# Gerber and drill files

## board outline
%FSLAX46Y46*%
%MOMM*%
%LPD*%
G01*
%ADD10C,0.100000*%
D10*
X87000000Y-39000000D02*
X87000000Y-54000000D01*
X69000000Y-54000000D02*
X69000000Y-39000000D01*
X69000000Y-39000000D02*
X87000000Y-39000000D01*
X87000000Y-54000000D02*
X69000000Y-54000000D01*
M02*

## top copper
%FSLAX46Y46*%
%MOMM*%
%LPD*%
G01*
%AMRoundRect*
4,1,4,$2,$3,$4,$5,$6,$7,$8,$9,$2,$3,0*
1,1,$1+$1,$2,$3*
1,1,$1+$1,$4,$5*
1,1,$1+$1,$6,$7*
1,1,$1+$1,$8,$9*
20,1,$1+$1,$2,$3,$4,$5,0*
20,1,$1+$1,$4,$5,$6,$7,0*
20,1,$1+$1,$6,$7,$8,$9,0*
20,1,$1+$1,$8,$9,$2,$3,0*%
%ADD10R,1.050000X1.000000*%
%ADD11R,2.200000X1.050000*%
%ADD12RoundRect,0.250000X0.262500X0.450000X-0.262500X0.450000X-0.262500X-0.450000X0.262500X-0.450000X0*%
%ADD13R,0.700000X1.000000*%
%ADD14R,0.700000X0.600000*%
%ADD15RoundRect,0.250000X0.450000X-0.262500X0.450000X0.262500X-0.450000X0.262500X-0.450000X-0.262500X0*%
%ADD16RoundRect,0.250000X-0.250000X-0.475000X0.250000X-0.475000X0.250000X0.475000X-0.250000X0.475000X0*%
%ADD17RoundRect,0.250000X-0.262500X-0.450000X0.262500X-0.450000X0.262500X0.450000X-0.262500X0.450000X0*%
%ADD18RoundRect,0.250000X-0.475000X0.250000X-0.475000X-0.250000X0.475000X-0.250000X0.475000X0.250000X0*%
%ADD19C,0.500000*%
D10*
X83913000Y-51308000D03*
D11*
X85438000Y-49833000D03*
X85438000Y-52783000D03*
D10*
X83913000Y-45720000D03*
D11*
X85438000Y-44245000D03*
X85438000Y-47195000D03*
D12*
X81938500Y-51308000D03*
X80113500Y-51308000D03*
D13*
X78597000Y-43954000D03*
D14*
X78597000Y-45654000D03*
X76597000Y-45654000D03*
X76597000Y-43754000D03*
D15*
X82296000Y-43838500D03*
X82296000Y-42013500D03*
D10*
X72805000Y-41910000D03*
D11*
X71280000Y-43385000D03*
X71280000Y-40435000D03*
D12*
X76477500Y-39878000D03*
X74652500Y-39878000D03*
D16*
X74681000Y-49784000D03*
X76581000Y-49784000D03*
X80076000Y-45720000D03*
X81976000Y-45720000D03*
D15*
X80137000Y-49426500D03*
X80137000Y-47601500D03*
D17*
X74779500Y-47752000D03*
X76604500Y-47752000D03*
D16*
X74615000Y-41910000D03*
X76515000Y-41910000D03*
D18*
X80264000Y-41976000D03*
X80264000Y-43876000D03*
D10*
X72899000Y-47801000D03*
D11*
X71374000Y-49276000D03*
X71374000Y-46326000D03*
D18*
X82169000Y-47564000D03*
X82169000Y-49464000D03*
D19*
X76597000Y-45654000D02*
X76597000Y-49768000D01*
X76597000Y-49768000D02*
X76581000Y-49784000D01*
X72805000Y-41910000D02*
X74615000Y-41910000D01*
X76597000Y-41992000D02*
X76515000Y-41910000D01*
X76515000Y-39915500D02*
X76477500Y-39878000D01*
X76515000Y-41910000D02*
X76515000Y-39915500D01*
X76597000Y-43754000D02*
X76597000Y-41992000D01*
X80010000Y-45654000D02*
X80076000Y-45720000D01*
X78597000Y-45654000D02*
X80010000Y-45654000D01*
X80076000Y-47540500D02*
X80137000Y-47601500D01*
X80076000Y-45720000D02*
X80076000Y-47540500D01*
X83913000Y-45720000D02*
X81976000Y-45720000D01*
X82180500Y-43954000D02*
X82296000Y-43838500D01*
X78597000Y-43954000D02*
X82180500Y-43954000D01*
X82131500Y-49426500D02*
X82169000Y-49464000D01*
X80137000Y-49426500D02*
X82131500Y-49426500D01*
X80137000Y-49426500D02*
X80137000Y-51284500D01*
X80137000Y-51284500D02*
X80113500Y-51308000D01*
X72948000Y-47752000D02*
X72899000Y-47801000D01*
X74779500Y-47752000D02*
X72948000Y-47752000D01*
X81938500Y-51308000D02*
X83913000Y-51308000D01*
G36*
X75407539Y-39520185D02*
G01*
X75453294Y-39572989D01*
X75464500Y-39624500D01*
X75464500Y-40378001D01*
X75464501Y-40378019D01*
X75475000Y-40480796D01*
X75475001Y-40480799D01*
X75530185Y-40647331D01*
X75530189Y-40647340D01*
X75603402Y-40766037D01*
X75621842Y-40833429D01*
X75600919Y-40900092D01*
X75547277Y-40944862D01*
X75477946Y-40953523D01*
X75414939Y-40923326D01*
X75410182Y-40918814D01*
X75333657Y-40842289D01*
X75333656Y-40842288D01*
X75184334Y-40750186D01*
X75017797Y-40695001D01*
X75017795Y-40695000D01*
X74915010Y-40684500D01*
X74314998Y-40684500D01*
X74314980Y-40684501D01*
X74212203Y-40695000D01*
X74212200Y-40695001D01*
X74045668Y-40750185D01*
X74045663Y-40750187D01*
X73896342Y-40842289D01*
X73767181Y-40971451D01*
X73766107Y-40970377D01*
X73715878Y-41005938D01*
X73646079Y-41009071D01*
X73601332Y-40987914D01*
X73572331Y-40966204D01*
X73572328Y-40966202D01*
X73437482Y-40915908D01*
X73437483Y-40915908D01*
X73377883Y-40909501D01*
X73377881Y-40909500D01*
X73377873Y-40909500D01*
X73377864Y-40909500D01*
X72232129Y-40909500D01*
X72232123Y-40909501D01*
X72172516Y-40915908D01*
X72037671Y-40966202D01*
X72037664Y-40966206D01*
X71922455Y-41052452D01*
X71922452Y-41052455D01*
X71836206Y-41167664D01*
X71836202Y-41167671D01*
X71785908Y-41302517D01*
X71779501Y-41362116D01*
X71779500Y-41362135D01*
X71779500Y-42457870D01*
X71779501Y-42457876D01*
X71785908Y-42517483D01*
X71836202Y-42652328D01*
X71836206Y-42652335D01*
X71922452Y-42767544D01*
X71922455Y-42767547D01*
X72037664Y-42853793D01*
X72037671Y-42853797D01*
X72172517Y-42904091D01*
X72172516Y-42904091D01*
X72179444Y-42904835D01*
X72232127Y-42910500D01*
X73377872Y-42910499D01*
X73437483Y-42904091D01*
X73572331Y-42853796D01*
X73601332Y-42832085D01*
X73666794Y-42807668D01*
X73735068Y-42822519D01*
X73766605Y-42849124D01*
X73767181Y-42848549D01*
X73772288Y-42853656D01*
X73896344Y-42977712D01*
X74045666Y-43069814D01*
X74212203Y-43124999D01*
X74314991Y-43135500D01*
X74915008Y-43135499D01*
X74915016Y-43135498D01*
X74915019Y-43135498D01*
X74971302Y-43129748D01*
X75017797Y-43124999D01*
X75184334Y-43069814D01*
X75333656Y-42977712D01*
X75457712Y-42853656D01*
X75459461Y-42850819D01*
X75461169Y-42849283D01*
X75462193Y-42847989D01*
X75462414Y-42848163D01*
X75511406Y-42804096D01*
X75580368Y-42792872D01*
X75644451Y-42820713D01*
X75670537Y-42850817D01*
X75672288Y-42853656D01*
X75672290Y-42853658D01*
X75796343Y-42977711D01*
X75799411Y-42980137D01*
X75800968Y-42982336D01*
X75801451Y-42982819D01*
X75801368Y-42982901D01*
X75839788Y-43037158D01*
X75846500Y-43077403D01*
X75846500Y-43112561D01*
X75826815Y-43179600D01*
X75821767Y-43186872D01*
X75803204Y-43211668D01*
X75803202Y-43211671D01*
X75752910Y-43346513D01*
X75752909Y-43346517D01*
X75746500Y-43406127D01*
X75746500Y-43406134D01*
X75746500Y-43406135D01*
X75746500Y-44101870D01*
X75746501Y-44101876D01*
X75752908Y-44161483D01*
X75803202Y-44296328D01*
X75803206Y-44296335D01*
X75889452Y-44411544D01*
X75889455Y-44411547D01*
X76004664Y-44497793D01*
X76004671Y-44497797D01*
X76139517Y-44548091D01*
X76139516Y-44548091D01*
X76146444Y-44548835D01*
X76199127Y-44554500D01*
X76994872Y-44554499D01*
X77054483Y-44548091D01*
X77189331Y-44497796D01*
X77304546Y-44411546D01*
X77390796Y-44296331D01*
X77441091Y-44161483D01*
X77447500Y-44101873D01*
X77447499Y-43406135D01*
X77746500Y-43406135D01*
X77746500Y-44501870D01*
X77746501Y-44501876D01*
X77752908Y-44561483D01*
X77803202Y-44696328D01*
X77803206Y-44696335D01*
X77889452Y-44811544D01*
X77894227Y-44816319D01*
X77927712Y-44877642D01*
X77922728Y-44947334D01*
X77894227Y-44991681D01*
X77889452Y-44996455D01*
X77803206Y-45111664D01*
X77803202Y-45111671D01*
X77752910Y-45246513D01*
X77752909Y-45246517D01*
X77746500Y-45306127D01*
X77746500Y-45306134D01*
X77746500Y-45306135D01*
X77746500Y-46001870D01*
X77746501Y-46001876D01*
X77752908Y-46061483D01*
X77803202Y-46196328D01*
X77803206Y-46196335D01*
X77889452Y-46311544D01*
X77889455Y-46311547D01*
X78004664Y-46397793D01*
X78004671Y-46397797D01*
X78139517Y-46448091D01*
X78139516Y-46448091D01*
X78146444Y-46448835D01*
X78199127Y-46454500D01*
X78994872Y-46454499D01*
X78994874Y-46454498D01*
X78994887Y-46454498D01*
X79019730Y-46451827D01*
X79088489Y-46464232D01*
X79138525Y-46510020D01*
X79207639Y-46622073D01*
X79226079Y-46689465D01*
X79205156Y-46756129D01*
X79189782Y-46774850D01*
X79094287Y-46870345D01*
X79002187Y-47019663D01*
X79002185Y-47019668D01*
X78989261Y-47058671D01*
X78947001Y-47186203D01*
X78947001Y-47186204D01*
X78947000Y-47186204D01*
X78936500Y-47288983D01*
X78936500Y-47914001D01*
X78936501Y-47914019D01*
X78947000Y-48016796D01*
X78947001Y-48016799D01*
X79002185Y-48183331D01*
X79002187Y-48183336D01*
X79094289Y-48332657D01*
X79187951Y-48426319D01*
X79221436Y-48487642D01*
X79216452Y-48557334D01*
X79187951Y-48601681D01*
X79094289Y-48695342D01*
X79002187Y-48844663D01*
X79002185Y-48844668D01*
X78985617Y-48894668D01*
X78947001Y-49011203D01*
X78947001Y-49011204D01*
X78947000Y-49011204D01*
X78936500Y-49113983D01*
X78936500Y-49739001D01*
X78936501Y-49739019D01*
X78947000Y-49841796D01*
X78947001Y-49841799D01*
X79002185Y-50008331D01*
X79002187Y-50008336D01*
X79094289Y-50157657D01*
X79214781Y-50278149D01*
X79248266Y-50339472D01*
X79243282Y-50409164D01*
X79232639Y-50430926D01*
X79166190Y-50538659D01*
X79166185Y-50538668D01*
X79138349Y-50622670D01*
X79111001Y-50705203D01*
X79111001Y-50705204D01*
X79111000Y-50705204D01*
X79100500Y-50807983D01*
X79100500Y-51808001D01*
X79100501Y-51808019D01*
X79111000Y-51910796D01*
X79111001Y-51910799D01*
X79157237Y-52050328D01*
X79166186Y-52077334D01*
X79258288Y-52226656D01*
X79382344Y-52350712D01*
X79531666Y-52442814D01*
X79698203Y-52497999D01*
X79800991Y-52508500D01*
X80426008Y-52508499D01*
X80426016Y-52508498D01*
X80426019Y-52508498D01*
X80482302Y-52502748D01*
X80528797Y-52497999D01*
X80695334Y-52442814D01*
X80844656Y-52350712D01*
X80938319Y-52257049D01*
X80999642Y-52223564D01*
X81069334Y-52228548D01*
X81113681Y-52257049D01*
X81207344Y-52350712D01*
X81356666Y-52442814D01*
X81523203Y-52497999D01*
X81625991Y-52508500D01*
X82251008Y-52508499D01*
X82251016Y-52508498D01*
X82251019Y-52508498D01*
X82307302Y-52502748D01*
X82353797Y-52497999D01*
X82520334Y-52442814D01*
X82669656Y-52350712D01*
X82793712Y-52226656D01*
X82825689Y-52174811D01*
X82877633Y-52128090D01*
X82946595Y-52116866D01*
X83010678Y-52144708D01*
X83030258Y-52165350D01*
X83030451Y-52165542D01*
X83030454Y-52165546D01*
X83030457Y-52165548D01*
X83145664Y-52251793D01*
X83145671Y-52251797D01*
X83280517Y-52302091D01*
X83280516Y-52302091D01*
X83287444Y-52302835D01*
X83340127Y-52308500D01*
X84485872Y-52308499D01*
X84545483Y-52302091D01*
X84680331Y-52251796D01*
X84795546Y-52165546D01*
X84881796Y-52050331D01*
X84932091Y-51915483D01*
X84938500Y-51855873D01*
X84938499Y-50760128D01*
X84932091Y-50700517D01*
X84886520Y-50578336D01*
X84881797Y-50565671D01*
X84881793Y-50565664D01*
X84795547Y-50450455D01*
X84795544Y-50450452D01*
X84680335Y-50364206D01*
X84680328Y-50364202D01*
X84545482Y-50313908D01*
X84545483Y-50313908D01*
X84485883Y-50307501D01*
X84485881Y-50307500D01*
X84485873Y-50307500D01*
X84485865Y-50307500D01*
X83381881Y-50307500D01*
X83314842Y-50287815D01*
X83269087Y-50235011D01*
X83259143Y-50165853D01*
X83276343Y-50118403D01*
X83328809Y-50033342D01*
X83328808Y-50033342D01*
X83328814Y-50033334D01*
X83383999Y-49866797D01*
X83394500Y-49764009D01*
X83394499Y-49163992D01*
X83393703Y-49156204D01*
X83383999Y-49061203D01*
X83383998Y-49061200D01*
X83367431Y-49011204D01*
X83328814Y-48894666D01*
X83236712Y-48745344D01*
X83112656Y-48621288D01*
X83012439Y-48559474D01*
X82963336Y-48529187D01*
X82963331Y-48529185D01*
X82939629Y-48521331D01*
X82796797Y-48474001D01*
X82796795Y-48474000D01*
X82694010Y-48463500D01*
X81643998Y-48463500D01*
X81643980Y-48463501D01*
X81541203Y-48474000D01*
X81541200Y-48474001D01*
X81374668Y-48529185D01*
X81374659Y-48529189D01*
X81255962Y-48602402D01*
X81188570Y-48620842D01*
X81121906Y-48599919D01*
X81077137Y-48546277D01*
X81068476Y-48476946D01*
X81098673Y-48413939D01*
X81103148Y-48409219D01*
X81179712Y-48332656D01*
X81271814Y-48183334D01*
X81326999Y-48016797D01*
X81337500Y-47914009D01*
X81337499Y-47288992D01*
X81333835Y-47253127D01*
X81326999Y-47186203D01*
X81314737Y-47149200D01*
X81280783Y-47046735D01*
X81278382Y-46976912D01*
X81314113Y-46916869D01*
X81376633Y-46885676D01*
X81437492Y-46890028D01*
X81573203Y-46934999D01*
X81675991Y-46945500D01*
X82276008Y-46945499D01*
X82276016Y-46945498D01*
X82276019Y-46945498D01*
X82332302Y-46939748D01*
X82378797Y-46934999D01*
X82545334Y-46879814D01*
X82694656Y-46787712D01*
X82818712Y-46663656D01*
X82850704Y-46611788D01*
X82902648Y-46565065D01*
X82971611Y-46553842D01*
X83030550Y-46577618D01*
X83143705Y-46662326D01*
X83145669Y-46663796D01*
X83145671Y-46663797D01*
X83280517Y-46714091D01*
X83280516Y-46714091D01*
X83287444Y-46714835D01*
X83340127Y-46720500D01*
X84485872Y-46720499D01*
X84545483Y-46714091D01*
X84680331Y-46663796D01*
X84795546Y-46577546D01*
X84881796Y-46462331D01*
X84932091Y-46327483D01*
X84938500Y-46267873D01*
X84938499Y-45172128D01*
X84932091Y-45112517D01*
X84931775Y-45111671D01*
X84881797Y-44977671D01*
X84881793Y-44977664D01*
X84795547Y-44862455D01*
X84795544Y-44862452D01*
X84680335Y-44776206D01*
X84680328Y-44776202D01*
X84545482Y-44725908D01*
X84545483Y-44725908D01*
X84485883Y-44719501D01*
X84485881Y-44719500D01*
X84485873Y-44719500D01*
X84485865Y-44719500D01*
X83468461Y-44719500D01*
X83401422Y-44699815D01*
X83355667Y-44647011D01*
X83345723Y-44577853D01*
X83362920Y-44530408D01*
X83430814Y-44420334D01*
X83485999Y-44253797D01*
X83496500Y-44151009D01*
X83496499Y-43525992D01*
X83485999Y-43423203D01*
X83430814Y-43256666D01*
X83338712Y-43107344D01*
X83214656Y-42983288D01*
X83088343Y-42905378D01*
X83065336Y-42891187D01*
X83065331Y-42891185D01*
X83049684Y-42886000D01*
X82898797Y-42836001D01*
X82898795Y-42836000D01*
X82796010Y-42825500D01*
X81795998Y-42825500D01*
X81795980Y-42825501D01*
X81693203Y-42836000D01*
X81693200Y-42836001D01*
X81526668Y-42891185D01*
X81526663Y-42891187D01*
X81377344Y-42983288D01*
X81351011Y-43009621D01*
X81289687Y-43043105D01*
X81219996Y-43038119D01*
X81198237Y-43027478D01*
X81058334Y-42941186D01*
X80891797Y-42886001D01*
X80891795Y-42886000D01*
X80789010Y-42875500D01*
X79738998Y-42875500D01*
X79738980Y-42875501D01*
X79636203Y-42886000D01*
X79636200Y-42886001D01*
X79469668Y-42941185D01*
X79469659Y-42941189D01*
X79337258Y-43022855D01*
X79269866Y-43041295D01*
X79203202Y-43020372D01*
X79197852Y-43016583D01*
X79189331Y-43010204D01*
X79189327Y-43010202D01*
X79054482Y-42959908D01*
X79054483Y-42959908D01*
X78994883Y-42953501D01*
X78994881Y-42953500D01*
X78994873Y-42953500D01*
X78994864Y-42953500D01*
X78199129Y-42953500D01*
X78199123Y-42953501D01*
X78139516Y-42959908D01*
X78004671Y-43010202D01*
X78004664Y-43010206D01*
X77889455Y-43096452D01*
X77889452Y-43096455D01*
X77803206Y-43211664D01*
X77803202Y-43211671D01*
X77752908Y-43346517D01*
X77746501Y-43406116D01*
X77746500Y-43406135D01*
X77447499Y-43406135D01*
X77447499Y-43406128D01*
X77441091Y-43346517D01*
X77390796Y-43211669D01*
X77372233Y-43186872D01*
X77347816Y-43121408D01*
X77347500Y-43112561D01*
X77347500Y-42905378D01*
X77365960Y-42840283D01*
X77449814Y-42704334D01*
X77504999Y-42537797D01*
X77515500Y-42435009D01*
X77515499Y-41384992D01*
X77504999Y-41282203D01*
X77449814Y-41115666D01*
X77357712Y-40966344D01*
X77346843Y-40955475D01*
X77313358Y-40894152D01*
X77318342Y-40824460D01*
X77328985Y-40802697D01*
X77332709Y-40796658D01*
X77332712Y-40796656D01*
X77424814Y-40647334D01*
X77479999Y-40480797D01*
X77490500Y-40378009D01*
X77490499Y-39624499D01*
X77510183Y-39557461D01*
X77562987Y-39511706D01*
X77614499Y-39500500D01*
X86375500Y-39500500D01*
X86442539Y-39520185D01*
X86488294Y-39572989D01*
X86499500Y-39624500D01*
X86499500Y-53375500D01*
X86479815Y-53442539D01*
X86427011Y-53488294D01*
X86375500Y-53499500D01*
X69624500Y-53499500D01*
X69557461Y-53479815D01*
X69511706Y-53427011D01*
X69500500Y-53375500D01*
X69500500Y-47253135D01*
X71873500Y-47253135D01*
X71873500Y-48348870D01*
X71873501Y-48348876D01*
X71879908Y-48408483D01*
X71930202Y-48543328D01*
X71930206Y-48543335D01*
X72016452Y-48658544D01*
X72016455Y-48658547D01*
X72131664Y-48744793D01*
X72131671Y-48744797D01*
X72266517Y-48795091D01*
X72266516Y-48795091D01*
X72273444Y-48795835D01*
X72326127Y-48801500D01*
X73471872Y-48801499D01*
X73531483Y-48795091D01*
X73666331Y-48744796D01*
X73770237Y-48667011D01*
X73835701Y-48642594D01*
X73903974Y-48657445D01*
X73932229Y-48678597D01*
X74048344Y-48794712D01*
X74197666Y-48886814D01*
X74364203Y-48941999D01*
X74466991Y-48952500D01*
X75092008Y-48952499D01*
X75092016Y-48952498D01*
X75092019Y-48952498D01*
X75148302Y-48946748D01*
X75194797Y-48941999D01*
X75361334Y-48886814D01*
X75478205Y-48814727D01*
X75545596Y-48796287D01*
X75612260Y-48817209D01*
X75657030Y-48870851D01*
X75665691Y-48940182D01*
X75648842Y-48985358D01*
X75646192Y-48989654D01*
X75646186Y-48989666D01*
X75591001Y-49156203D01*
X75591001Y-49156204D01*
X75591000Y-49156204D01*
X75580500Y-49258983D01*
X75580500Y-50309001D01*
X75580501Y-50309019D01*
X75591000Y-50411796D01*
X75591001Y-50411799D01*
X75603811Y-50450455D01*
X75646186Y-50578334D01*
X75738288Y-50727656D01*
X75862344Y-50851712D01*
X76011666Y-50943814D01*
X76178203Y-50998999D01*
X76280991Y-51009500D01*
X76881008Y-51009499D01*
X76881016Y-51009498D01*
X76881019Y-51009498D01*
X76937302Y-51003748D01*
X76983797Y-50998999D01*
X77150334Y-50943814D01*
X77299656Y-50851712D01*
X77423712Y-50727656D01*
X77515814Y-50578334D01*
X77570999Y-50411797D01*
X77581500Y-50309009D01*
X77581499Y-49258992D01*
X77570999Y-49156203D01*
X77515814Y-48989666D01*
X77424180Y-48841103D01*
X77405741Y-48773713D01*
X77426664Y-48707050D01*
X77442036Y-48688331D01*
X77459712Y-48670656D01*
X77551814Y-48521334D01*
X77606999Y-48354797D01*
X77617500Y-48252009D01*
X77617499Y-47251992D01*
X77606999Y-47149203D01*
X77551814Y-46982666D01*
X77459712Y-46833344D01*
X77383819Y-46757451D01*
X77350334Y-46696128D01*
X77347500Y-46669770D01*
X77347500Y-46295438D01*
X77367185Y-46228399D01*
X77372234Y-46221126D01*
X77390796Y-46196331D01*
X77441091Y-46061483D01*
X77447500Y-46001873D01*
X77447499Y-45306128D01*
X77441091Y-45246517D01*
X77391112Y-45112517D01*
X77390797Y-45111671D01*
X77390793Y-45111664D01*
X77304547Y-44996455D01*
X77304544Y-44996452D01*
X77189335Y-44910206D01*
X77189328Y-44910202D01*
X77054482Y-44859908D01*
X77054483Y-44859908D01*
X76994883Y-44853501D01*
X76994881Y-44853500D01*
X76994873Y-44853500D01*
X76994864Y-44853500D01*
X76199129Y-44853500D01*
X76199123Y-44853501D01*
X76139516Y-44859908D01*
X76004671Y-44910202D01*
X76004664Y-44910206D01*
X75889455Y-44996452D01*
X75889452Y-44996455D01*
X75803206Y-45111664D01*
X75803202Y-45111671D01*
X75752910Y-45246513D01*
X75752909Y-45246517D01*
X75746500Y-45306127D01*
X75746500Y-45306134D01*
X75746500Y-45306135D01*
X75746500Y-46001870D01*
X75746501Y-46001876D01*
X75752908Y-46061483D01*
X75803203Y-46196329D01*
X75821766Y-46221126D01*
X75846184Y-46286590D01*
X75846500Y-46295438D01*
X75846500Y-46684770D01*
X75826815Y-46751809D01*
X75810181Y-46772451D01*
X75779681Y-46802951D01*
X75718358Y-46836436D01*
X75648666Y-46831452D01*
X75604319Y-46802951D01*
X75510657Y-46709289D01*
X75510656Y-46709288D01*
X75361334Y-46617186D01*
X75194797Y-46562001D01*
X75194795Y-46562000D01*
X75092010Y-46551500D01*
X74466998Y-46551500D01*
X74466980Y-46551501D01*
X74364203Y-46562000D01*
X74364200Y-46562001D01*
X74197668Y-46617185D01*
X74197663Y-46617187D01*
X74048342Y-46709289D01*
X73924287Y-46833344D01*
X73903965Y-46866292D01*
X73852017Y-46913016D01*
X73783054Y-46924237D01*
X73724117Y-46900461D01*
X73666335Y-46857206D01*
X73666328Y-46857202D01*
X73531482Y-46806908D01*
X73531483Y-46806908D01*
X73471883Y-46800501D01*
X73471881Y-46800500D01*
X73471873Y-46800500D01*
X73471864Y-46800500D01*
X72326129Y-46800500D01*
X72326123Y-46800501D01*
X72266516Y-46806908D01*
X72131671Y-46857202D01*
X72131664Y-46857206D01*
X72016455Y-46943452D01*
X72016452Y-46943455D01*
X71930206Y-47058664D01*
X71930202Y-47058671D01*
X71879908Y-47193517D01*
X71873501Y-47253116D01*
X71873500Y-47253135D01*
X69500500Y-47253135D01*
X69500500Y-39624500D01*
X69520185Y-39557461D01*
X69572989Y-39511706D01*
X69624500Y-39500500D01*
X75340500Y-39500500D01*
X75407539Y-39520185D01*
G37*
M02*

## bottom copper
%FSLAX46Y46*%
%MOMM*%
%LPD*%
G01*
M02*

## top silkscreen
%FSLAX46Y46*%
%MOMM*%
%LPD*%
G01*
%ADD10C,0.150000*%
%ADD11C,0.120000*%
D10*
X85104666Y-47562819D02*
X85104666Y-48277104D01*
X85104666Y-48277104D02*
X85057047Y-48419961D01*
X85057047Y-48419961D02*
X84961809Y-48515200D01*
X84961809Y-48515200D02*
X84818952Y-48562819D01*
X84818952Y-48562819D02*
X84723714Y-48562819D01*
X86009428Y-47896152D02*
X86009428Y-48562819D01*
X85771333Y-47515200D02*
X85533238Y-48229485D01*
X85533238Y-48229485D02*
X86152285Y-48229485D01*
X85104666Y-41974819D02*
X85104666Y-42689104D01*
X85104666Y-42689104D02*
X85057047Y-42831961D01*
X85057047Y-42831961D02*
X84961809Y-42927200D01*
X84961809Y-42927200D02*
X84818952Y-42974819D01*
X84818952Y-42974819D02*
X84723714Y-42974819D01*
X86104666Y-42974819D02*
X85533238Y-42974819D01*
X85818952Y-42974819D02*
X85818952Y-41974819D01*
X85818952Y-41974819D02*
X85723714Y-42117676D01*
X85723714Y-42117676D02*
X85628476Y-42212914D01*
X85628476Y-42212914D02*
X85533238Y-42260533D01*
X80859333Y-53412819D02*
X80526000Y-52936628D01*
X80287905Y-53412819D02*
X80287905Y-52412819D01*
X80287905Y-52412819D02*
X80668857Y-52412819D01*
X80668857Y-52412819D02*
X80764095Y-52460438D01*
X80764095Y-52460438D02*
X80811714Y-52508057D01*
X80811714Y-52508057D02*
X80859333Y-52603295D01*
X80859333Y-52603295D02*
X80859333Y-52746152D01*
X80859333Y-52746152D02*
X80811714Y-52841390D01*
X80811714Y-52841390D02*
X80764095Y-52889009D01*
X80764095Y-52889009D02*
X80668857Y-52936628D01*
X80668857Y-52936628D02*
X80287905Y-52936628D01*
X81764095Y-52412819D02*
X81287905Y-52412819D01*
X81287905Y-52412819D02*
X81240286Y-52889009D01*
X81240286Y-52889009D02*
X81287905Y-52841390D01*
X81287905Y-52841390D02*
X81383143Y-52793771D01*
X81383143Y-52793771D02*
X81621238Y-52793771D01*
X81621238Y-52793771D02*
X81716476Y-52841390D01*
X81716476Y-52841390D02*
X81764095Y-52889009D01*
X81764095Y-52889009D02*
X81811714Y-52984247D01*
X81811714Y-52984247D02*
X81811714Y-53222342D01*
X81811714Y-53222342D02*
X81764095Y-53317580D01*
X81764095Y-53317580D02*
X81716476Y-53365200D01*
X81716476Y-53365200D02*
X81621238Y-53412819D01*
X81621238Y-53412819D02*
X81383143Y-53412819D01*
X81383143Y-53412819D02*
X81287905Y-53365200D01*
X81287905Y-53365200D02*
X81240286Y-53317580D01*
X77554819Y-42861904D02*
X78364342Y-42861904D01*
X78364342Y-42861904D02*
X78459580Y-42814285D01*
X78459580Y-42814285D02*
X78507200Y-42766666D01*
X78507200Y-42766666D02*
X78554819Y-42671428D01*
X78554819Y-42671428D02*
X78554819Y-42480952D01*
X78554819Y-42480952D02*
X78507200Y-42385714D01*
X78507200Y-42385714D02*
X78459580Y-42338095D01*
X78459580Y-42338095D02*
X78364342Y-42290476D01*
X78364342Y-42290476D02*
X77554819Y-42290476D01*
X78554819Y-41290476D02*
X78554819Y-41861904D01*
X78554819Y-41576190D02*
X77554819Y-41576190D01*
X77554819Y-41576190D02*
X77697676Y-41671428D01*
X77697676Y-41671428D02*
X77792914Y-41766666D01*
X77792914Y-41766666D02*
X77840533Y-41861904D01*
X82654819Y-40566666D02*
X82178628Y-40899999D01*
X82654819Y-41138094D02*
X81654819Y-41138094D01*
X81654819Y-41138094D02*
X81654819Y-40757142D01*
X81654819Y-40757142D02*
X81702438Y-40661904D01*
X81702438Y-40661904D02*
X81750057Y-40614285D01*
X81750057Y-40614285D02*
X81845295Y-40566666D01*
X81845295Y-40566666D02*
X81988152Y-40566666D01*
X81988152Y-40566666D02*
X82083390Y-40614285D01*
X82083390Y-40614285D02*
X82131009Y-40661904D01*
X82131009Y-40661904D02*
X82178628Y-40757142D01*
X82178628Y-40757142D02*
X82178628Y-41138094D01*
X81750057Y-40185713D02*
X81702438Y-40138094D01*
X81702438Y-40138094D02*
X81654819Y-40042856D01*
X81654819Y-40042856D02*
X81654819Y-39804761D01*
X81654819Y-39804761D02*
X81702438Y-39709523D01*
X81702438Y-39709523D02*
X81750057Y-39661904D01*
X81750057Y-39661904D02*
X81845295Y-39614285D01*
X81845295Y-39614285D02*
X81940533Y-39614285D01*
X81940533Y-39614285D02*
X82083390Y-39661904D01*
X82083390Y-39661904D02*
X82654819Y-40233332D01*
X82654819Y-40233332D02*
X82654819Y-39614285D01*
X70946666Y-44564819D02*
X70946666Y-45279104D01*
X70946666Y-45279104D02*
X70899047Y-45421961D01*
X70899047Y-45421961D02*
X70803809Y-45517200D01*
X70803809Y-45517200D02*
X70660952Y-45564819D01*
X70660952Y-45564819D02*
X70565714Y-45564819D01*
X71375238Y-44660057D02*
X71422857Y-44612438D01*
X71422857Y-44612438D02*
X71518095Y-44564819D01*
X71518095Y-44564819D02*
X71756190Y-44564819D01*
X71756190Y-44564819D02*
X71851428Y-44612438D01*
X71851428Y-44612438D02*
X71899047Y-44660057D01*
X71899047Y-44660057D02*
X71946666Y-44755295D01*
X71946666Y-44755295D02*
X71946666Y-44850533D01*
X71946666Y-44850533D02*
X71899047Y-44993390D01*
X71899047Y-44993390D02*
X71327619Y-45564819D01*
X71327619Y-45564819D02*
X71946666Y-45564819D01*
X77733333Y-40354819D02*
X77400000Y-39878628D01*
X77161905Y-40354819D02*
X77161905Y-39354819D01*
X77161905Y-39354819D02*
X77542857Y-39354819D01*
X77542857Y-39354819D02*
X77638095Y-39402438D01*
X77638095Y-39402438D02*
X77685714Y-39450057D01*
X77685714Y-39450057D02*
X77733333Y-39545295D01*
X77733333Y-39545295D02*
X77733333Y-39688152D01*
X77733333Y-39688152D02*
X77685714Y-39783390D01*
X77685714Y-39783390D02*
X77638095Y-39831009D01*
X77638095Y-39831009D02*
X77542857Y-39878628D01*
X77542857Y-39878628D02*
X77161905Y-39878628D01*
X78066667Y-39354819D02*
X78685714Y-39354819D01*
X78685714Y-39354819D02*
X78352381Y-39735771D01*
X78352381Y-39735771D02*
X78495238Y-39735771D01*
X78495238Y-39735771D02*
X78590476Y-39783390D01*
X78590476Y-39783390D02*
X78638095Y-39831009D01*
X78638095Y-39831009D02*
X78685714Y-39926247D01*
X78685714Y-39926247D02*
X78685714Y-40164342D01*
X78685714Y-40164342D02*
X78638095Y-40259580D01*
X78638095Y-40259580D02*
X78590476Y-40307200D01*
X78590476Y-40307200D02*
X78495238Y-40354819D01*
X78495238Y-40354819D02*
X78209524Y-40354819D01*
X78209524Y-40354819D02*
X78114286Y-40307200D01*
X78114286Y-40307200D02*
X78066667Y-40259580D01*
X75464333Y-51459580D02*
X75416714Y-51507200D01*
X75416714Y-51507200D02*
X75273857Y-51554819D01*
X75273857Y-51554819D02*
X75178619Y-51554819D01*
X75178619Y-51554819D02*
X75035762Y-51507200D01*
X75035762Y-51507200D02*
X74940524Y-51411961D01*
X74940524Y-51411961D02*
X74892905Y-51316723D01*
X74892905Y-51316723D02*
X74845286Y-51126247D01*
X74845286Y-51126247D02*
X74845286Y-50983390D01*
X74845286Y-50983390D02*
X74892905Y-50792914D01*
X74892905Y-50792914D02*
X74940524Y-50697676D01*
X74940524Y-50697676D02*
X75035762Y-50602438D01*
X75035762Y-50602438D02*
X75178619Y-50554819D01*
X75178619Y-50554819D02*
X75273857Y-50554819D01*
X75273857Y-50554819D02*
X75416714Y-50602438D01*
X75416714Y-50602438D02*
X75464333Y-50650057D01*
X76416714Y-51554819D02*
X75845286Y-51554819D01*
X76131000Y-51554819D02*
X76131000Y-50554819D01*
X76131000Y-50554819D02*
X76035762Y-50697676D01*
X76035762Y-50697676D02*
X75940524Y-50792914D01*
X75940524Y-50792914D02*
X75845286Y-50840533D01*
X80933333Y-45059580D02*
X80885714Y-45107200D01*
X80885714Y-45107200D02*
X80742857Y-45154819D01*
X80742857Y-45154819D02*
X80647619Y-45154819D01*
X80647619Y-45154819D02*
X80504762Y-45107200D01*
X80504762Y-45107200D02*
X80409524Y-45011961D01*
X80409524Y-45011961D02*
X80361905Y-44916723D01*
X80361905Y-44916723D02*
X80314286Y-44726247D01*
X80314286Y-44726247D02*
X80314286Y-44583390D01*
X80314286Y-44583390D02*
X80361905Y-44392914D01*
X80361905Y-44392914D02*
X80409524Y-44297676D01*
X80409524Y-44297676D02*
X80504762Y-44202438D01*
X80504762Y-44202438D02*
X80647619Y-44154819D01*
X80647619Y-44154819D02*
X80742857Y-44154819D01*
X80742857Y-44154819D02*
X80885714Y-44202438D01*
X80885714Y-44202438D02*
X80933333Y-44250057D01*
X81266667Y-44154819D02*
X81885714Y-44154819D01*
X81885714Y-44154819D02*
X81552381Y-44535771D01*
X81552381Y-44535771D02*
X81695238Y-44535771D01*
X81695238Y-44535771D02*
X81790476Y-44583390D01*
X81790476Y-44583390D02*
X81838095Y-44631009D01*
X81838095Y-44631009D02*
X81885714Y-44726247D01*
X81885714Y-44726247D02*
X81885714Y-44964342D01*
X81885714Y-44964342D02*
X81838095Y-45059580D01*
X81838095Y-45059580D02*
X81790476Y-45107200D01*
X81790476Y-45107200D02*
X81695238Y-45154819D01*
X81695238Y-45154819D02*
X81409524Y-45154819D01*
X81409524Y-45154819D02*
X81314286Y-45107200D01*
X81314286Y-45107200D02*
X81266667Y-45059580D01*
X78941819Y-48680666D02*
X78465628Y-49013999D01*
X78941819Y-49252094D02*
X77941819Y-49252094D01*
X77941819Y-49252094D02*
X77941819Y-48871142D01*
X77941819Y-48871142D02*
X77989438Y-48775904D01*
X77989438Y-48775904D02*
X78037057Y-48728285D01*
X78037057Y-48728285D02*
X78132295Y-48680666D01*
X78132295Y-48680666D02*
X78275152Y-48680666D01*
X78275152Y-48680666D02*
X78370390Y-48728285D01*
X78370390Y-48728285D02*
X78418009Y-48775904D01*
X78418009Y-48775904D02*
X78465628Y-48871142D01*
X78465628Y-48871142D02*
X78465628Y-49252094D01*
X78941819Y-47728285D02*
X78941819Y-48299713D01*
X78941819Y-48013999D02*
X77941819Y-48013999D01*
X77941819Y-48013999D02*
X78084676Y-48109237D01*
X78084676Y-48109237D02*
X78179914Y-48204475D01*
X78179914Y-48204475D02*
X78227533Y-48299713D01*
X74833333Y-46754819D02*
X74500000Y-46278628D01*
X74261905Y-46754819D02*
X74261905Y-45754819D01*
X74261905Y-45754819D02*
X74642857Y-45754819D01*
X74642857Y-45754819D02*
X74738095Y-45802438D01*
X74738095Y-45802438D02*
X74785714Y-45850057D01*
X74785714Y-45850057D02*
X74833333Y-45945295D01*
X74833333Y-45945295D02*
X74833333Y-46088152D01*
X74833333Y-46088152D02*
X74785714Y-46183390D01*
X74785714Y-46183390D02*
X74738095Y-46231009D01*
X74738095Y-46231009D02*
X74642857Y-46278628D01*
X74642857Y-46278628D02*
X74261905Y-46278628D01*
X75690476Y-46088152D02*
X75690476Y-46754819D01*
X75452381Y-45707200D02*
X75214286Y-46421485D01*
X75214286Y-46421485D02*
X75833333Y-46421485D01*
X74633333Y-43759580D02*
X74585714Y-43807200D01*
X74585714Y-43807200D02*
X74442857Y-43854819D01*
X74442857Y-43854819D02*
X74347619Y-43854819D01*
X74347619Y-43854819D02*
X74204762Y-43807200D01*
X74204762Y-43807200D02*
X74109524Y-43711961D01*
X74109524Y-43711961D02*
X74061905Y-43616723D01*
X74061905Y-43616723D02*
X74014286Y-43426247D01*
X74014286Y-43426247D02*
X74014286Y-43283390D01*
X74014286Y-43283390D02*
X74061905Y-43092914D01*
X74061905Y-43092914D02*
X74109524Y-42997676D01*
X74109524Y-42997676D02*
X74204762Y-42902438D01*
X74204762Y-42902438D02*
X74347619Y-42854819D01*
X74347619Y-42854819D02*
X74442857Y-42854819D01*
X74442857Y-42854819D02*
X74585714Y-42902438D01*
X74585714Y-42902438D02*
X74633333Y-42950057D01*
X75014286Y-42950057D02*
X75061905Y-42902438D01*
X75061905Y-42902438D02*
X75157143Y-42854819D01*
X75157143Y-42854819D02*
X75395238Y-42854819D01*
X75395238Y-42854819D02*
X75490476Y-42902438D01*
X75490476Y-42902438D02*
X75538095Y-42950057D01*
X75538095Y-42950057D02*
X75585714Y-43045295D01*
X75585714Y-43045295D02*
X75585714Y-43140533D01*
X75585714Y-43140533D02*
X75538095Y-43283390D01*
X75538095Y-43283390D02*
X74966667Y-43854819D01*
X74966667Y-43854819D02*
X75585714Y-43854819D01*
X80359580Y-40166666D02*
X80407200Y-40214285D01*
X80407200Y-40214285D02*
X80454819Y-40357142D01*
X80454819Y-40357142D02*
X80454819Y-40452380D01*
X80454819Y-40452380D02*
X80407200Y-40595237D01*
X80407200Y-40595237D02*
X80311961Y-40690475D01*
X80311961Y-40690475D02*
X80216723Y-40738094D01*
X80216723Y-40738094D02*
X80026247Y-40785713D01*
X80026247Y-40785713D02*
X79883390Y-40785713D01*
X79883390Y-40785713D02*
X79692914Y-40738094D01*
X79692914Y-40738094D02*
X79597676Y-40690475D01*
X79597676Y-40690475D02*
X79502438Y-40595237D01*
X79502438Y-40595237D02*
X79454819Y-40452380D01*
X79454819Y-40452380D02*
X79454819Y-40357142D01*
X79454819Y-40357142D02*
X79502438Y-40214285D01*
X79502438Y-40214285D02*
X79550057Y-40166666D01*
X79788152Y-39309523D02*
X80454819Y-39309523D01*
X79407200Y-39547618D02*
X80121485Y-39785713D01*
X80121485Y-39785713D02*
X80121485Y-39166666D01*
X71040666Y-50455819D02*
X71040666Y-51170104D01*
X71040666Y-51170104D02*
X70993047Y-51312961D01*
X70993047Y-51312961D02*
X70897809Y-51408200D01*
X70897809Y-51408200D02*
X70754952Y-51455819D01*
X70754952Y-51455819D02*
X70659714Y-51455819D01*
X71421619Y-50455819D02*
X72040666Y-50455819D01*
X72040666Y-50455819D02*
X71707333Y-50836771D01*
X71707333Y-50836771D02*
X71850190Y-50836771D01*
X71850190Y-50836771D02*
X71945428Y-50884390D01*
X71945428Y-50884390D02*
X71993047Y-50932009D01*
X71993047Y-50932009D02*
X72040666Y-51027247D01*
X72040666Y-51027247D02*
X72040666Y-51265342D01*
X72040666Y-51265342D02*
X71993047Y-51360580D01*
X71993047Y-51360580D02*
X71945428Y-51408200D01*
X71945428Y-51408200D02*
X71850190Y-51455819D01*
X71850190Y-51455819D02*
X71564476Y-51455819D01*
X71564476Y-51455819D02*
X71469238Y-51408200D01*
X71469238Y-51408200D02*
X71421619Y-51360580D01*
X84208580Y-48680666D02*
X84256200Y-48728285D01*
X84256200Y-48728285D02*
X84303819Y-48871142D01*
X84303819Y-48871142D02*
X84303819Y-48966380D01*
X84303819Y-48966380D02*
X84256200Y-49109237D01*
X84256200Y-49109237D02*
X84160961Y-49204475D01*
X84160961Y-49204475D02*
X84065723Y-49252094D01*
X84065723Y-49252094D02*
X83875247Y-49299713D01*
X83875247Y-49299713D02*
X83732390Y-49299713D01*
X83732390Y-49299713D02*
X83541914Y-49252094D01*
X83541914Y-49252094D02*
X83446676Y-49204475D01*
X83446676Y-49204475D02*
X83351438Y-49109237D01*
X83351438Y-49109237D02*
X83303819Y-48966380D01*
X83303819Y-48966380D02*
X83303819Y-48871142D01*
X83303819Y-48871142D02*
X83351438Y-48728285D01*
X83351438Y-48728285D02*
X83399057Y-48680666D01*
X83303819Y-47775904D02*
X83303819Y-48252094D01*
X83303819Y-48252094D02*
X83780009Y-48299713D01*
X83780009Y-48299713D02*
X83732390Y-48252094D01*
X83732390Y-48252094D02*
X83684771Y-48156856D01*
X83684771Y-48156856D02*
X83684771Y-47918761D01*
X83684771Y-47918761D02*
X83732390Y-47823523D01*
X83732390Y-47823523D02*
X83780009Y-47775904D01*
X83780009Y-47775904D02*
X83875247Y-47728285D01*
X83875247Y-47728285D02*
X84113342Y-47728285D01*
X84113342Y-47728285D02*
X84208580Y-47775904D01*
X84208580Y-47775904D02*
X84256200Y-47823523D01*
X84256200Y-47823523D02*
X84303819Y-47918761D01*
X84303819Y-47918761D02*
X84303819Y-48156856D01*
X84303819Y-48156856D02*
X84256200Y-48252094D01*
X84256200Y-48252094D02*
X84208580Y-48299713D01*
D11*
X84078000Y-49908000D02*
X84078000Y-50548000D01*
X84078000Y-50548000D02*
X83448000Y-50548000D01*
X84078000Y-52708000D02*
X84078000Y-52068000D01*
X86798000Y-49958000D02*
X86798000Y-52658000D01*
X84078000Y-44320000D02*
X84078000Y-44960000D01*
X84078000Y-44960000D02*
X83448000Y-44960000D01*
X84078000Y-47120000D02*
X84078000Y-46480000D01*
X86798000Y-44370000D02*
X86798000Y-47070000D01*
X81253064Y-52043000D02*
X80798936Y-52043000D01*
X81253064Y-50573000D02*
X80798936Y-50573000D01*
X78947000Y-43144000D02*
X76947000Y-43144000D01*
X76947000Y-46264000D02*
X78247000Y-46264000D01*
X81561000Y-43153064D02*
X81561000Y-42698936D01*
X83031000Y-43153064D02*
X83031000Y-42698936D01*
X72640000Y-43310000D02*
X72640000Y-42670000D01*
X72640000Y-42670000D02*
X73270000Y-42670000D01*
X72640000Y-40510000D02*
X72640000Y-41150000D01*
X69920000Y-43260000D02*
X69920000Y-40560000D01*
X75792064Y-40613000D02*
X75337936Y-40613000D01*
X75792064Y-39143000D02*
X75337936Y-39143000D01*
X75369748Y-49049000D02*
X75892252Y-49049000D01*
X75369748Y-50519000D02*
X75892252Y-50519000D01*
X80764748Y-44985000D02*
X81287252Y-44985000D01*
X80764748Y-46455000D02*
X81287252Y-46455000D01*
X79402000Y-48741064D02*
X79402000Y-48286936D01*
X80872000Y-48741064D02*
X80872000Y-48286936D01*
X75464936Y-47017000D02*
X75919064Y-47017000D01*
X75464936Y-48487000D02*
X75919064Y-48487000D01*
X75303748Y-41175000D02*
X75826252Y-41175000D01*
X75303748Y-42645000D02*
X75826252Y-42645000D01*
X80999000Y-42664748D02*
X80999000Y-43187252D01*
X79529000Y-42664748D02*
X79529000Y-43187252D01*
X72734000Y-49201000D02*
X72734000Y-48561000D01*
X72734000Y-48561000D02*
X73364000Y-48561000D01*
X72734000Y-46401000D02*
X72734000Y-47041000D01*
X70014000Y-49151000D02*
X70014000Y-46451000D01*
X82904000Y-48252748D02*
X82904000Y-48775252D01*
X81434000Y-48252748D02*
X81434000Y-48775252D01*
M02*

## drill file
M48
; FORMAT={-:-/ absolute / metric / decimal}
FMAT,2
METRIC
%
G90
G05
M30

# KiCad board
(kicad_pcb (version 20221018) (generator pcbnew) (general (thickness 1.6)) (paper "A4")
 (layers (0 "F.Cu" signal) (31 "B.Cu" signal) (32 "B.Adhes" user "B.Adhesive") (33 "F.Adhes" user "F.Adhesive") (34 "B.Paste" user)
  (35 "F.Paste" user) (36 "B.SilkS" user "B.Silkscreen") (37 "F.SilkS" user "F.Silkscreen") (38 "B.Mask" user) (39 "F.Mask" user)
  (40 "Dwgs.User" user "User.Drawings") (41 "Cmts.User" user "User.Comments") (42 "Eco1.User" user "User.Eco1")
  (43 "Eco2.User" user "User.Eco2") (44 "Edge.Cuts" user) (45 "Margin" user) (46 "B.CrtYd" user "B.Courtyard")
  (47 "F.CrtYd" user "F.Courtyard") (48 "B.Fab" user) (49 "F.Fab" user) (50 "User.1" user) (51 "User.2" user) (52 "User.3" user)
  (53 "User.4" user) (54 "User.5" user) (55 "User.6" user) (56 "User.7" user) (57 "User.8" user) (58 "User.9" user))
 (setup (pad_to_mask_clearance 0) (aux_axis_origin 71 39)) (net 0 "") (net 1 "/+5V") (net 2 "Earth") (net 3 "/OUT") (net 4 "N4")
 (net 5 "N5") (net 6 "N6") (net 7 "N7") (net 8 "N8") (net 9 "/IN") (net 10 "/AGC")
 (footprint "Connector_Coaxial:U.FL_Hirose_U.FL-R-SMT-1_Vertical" (layer "F.Cu") (at 84.963 51.308)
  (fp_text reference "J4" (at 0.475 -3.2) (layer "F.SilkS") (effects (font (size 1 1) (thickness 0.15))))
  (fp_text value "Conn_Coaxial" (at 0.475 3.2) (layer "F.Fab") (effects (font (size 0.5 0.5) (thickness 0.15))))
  (fp_line (start -0.885 -1.4) (end -0.885 -0.76) (stroke (width 0.12) (type solid)) (layer "F.SilkS"))
  (fp_line (start -0.885 -0.76) (end -1.515 -0.76) (stroke (width 0.12) (type solid)) (layer "F.SilkS"))
  (fp_line (start -0.885 1.4) (end -0.885 0.76) (stroke (width 0.12) (type solid)) (layer "F.SilkS"))
  (fp_line (start 1.835 -1.35) (end 1.835 1.35) (stroke (width 0.12) (type solid)) (layer "F.SilkS"))
  (pad "1" smd rect (at -1.05 0) (size 1.05 1) (layers "F.Cu" "F.Paste" "F.Mask") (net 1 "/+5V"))
  (pad "2" smd rect (at 0.475 -1.475) (size 2.2 1.05) (layers "F.Cu" "F.Paste" "F.Mask") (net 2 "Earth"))
  (pad "2" smd rect (at 0.475 1.475) (size 2.2 1.05) (layers "F.Cu" "F.Paste" "F.Mask") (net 2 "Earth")))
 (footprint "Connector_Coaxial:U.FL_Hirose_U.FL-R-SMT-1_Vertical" (layer "F.Cu") (at 84.963 45.72)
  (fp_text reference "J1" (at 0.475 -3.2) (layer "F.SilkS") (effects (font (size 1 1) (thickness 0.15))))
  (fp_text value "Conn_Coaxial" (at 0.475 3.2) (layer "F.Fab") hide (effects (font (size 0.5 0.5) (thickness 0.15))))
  (fp_line (start -0.885 -1.4) (end -0.885 -0.76) (stroke (width 0.12) (type solid)) (layer "F.SilkS"))
  (fp_line (start -0.885 -0.76) (end -1.515 -0.76) (stroke (width 0.12) (type solid)) (layer "F.SilkS"))
  (fp_line (start -0.885 1.4) (end -0.885 0.76) (stroke (width 0.12) (type solid)) (layer "F.SilkS"))
  (fp_line (start 1.835 -1.35) (end 1.835 1.35) (stroke (width 0.12) (type solid)) (layer "F.SilkS"))
  (pad "1" smd rect (at -1.05 0) (size 1.05 1) (layers "F.Cu" "F.Paste" "F.Mask") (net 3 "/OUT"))
  (pad "2" smd rect (at 0.475 -1.475) (size 2.2 1.05) (layers "F.Cu" "F.Paste" "F.Mask") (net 2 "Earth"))
  (pad "2" smd rect (at 0.475 1.475) (size 2.2 1.05) (layers "F.Cu" "F.Paste" "F.Mask") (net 2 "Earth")))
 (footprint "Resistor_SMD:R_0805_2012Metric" (layer "F.Cu") (at 81.026 51.308 180)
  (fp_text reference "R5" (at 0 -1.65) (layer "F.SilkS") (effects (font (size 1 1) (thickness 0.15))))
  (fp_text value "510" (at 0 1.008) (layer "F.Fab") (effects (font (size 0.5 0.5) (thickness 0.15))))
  (fp_line (start -0.227064 -0.735) (end 0.227064 -0.735) (stroke (width 0.12) (type solid)) (layer "F.SilkS"))
  (fp_line (start -0.227064 0.735) (end 0.227064 0.735) (stroke (width 0.12) (type solid)) (layer "F.SilkS"))
  (pad "1" smd roundrect (at -0.9125 0 180) (size 1.025 1.4) (layers "F.Cu" "F.Paste" "F.Mask") (roundrect_rratio 0.243902439)
   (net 1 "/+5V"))
  (pad "2" smd roundrect (at 0.9125 0 180) (size 1.025 1.4) (layers "F.Cu" "F.Paste" "F.Mask") (roundrect_rratio 0.243902439) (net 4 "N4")))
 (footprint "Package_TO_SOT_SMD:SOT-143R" (layer "F.Cu") (at 77.597 44.704 -90)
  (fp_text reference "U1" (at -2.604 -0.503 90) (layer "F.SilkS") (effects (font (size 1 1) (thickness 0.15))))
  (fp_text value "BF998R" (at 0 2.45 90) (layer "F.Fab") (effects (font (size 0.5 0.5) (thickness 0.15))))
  (fp_line (start -1.56 -1.35) (end -1.56 0.65) (stroke (width 0.12) (type solid)) (layer "F.SilkS"))
  (fp_line (start 1.56 0.65) (end 1.56 -0.65) (stroke (width 0.12) (type solid)) (layer "F.SilkS"))
  (pad "1" smd rect (at -0.75 -1 180) (size 0.7 1) (layers "F.Cu" "F.Paste" "F.Mask") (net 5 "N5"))
  (pad "2" smd rect (at 0.95 -1 180) (size 0.7 0.6) (layers "F.Cu" "F.Paste" "F.Mask") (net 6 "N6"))
  (pad "3" smd rect (at 0.95 1 180) (size 0.7 0.6) (layers "F.Cu" "F.Paste" "F.Mask") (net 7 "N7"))
  (pad "4" smd rect (at -0.95 1 180) (size 0.7 0.6) (layers "F.Cu" "F.Paste" "F.Mask") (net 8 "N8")))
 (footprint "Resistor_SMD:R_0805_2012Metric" (layer "F.Cu") (at 82.296 42.926 90)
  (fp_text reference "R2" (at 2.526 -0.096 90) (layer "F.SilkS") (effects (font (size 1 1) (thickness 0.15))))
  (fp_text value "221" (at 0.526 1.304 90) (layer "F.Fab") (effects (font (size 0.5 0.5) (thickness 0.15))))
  (fp_line (start -0.227064 -0.735) (end 0.227064 -0.735) (stroke (width 0.12) (type solid)) (layer "F.SilkS"))
  (fp_line (start -0.227064 0.735) (end 0.227064 0.735) (stroke (width 0.12) (type solid)) (layer "F.SilkS"))
  (pad "1" smd roundrect (at -0.9125 0 90) (size 1.025 1.4) (layers "F.Cu" "F.Paste" "F.Mask") (roundrect_rratio 0.243902439) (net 5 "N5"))
  (pad "2" smd roundrect (at 0.9125 0 90) (size 1.025 1.4) (layers "F.Cu" "F.Paste" "F.Mask") (roundrect_rratio 0.243902439) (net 2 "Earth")))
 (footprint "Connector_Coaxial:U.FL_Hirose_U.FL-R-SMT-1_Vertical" (layer "F.Cu") (at 71.755 41.91 180)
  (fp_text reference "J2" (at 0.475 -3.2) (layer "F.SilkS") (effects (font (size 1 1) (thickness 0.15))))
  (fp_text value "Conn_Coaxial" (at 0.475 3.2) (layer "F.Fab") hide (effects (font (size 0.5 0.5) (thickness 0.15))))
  (fp_line (start -0.885 -1.4) (end -0.885 -0.76) (stroke (width 0.12) (type solid)) (layer "F.SilkS"))
  (fp_line (start -0.885 -0.76) (end -1.515 -0.76) (stroke (width 0.12) (type solid)) (layer "F.SilkS"))
  (fp_line (start -0.885 1.4) (end -0.885 0.76) (stroke (width 0.12) (type solid)) (layer "F.SilkS"))
  (fp_line (start 1.835 -1.35) (end 1.835 1.35) (stroke (width 0.12) (type solid)) (layer "F.SilkS"))
  (pad "1" smd rect (at -1.05 0 180) (size 1.05 1) (layers "F.Cu" "F.Paste" "F.Mask") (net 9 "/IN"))
  (pad "2" smd rect (at 0.475 -1.475 180) (size 2.2 1.05) (layers "F.Cu" "F.Paste" "F.Mask") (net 2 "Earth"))
  (pad "2" smd rect (at 0.475 1.475 180) (size 2.2 1.05) (layers "F.Cu" "F.Paste" "F.Mask") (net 2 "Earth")))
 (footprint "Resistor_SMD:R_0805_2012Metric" (layer "F.Cu") (at 75.565 39.878 180)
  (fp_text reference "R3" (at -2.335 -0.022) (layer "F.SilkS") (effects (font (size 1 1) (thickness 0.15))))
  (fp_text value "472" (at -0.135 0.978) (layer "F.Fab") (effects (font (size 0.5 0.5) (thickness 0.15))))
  (fp_line (start -0.227064 -0.735) (end 0.227064 -0.735) (stroke (width 0.12) (type solid)) (layer "F.SilkS"))
  (fp_line (start -0.227064 0.735) (end 0.227064 0.735) (stroke (width 0.12) (type solid)) (layer "F.SilkS"))
  (pad "1" smd roundrect (at -0.9125 0 180) (size 1.025 1.4) (layers "F.Cu" "F.Paste" "F.Mask") (roundrect_rratio 0.243902439) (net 8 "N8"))
  (pad "2" smd roundrect (at 0.9125 0 180) (size 1.025 1.4) (layers "F.Cu" "F.Paste" "F.Mask") (roundrect_rratio 0.243902439)
   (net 2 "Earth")))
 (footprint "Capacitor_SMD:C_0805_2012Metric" (layer "F.Cu") (at 75.631 49.784)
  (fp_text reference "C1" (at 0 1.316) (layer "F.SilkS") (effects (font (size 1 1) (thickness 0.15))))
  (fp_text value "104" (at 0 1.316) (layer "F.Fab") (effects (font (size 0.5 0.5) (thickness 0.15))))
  (fp_line (start -0.261252 -0.735) (end 0.261252 -0.735) (stroke (width 0.12) (type solid)) (layer "F.SilkS"))
  (fp_line (start -0.261252 0.735) (end 0.261252 0.735) (stroke (width 0.12) (type solid)) (layer "F.SilkS"))
  (pad "1" smd roundrect (at -0.95 0) (size 1 1.45) (layers "F.Cu" "F.Paste" "F.Mask") (roundrect_rratio 0.25) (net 2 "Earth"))
  (pad "2" smd roundrect (at 0.95 0) (size 1 1.45) (layers "F.Cu" "F.Paste" "F.Mask") (roundrect_rratio 0.25) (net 7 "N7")))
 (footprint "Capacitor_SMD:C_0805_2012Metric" (layer "F.Cu") (at 81.026 45.72)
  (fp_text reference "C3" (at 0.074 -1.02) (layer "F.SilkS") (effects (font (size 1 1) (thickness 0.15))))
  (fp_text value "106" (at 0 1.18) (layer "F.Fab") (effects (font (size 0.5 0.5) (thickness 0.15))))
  (fp_line (start -0.261252 -0.735) (end 0.261252 -0.735) (stroke (width 0.12) (type solid)) (layer "F.SilkS"))
  (fp_line (start -0.261252 0.735) (end 0.261252 0.735) (stroke (width 0.12) (type solid)) (layer "F.SilkS"))
  (pad "1" smd roundrect (at -0.95 0) (size 1 1.45) (layers "F.Cu" "F.Paste" "F.Mask") (roundrect_rratio 0.25) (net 6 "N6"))
  (pad "2" smd roundrect (at 0.95 0) (size 1 1.45) (layers "F.Cu" "F.Paste" "F.Mask") (roundrect_rratio 0.25) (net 3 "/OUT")))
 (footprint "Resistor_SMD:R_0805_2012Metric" (layer "F.Cu") (at 80.137 48.514 90)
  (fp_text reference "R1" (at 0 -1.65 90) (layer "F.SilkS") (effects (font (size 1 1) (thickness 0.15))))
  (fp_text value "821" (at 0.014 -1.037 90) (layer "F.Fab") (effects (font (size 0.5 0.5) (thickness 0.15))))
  (fp_line (start -0.227064 -0.735) (end 0.227064 -0.735) (stroke (width 0.12) (type solid)) (layer "F.SilkS"))
  (fp_line (start -0.227064 0.735) (end 0.227064 0.735) (stroke (width 0.12) (type solid)) (layer "F.SilkS"))
  (pad "1" smd roundrect (at -0.9125 0 90) (size 1.025 1.4) (layers "F.Cu" "F.Paste" "F.Mask") (roundrect_rratio 0.243902439) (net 4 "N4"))
  (pad "2" smd roundrect (at 0.9125 0 90) (size 1.025 1.4) (layers "F.Cu" "F.Paste" "F.Mask") (roundrect_rratio 0.243902439) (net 6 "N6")))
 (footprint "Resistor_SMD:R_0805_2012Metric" (layer "F.Cu") (at 75.692 47.752)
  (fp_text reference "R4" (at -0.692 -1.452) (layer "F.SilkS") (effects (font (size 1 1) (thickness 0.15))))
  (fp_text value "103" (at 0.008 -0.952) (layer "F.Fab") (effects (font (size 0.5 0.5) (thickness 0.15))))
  (fp_line (start -0.227064 -0.735) (end 0.227064 -0.735) (stroke (width 0.12) (type solid)) (layer "F.SilkS"))
  (fp_line (start -0.227064 0.735) (end 0.227064 0.735) (stroke (width 0.12) (type solid)) (layer "F.SilkS"))
  (pad "1" smd roundrect (at -0.9125 0) (size 1.025 1.4) (layers "F.Cu" "F.Paste" "F.Mask") (roundrect_rratio 0.243902439) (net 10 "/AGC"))
  (pad "2" smd roundrect (at 0.9125 0) (size 1.025 1.4) (layers "F.Cu" "F.Paste" "F.Mask") (roundrect_rratio 0.243902439) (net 7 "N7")))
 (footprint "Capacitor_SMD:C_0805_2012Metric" (layer "F.Cu") (at 75.565 41.91)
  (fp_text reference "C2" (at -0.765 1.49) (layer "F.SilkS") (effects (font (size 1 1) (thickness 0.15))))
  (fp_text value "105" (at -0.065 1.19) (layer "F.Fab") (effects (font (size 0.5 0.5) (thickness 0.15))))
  (fp_line (start -0.261252 -0.735) (end 0.261252 -0.735) (stroke (width 0.12) (type solid)) (layer "F.SilkS"))
  (fp_line (start -0.261252 0.735) (end 0.261252 0.735) (stroke (width 0.12) (type solid)) (layer "F.SilkS"))
  (pad "1" smd roundrect (at -0.95 0) (size 1 1.45) (layers "F.Cu" "F.Paste" "F.Mask") (roundrect_rratio 0.25) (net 9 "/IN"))
  (pad "2" smd roundrect (at 0.95 0) (size 1 1.45) (layers "F.Cu" "F.Paste" "F.Mask") (roundrect_rratio 0.25) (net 8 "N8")))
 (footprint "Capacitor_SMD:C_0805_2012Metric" (layer "F.Cu") (at 80.264 42.926 -90)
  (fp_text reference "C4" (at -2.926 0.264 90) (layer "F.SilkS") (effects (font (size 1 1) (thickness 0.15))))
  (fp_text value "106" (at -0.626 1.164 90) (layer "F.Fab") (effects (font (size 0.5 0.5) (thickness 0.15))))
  (fp_line (start -0.261252 -0.735) (end 0.261252 -0.735) (stroke (width 0.12) (type solid)) (layer "F.SilkS"))
  (fp_line (start -0.261252 0.735) (end 0.261252 0.735) (stroke (width 0.12) (type solid)) (layer "F.SilkS"))
  (pad "1" smd roundrect (at -0.95 0 270) (size 1 1.45) (layers "F.Cu" "F.Paste" "F.Mask") (roundrect_rratio 0.25) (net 2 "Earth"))
  (pad "2" smd roundrect (at 0.95 0 270) (size 1 1.45) (layers "F.Cu" "F.Paste" "F.Mask") (roundrect_rratio 0.25) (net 5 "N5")))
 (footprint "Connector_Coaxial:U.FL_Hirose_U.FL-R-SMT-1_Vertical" (layer "F.Cu") (at 71.849 47.801 180)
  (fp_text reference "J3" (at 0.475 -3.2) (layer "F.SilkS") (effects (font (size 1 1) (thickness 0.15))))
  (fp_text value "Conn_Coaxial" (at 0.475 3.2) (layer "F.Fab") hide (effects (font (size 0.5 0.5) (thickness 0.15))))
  (fp_line (start -0.885 -1.4) (end -0.885 -0.76) (stroke (width 0.12) (type solid)) (layer "F.SilkS"))
  (fp_line (start -0.885 -0.76) (end -1.515 -0.76) (stroke (width 0.12) (type solid)) (layer "F.SilkS"))
  (fp_line (start -0.885 1.4) (end -0.885 0.76) (stroke (width 0.12) (type solid)) (layer "F.SilkS"))
  (fp_line (start 1.835 -1.35) (end 1.835 1.35) (stroke (width 0.12) (type solid)) (layer "F.SilkS"))
  (pad "1" smd rect (at -1.05 0 180) (size 1.05 1) (layers "F.Cu" "F.Paste" "F.Mask") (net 10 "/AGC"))
  (pad "2" smd rect (at 0.475 -1.475 180) (size 2.2 1.05) (layers "F.Cu" "F.Paste" "F.Mask") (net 2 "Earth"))
  (pad "2" smd rect (at 0.475 1.475 180) (size 2.2 1.05) (layers "F.Cu" "F.Paste" "F.Mask") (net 2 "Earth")))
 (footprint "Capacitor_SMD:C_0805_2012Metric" (layer "F.Cu") (at 82.169 48.514 -90)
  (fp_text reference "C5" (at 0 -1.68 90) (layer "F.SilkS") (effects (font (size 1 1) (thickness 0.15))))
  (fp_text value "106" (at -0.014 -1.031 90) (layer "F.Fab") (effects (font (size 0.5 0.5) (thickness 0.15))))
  (fp_line (start -0.261252 -0.735) (end 0.261252 -0.735) (stroke (width 0.12) (type solid)) (layer "F.SilkS"))
  (fp_line (start -0.261252 0.735) (end 0.261252 0.735) (stroke (width 0.12) (type solid)) (layer "F.SilkS"))
  (pad "1" smd roundrect (at -0.95 0 270) (size 1 1.45) (layers "F.Cu" "F.Paste" "F.Mask") (roundrect_rratio 0.25) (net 2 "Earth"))
  (pad "2" smd roundrect (at 0.95 0 270) (size 1 1.45) (layers "F.Cu" "F.Paste" "F.Mask") (roundrect_rratio 0.25) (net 4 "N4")))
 (gr_line (start 87 39) (end 87 54) (stroke (width 0.1) (type default)) (layer "Edge.Cuts"))
 (gr_line (start 69 54) (end 69 39) (stroke (width 0.1) (type default)) (layer "Edge.Cuts"))
 (gr_line (start 69 39) (end 87 39) (stroke (width 0.1) (type default)) (layer "Edge.Cuts"))
 (gr_line (start 87 54) (end 69 54) (stroke (width 0.1) (type default)) (layer "Edge.Cuts"))
 (segment (start 76.597 45.654) (end 76.597 49.768) (width 0.5) (layer "F.Cu") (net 7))
 (segment (start 76.597 49.768) (end 76.581 49.784) (width 0.5) (layer "F.Cu") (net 7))
 (segment (start 72.805 41.91) (end 74.615 41.91) (width 0.5) (layer "F.Cu") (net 9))
 (segment (start 76.597 41.992) (end 76.515 41.91) (width 0.5) (layer "F.Cu") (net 8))
 (segment (start 76.515 39.9155) (end 76.4775 39.878) (width 0.5) (layer "F.Cu") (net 8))
 (segment (start 76.515 41.91) (end 76.515 39.9155) (width 0.5) (layer "F.Cu") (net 8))
 (segment (start 76.597 43.754) (end 76.597 41.992) (width 0.5) (layer "F.Cu") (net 8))
 (segment (start 80.01 45.654) (end 80.076 45.72) (width 0.5) (layer "F.Cu") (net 6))
 (segment (start 78.597 45.654) (end 80.01 45.654) (width 0.5) (layer "F.Cu") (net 6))
 (segment (start 80.076 47.5405) (end 80.137 47.6015) (width 0.5) (layer "F.Cu") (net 6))
 (segment (start 80.076 45.72) (end 80.076 47.5405) (width 0.5) (layer "F.Cu") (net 6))
 (segment (start 83.913 45.72) (end 81.976 45.72) (width 0.5) (layer "F.Cu") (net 3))
 (segment (start 82.1805 43.954) (end 82.296 43.8385) (width 0.5) (layer "F.Cu") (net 5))
 (segment (start 78.597 43.954) (end 82.1805 43.954) (width 0.5) (layer "F.Cu") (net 5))
 (segment (start 82.1315 49.4265) (end 82.169 49.464) (width 0.5) (layer "F.Cu") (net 4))
 (segment (start 80.137 49.4265) (end 82.1315 49.4265) (width 0.5) (layer "F.Cu") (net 4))
 (segment (start 80.137 49.4265) (end 80.137 51.2845) (width 0.5) (layer "F.Cu") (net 4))
 (segment (start 80.137 51.2845) (end 80.1135 51.308) (width 0.5) (layer "F.Cu") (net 4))
 (segment (start 72.948 47.752) (end 72.899 47.801) (width 0.5) (layer "F.Cu") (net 10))
 (segment (start 74.7795 47.752) (end 72.948 47.752) (width 0.5) (layer "F.Cu") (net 10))
 (segment (start 81.9385 51.308) (end 83.913 51.308) (width 0.5) (layer "F.Cu") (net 1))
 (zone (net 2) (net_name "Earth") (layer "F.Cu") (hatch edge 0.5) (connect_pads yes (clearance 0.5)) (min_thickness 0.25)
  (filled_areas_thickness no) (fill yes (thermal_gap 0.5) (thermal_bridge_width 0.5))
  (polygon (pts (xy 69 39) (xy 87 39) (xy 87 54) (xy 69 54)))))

